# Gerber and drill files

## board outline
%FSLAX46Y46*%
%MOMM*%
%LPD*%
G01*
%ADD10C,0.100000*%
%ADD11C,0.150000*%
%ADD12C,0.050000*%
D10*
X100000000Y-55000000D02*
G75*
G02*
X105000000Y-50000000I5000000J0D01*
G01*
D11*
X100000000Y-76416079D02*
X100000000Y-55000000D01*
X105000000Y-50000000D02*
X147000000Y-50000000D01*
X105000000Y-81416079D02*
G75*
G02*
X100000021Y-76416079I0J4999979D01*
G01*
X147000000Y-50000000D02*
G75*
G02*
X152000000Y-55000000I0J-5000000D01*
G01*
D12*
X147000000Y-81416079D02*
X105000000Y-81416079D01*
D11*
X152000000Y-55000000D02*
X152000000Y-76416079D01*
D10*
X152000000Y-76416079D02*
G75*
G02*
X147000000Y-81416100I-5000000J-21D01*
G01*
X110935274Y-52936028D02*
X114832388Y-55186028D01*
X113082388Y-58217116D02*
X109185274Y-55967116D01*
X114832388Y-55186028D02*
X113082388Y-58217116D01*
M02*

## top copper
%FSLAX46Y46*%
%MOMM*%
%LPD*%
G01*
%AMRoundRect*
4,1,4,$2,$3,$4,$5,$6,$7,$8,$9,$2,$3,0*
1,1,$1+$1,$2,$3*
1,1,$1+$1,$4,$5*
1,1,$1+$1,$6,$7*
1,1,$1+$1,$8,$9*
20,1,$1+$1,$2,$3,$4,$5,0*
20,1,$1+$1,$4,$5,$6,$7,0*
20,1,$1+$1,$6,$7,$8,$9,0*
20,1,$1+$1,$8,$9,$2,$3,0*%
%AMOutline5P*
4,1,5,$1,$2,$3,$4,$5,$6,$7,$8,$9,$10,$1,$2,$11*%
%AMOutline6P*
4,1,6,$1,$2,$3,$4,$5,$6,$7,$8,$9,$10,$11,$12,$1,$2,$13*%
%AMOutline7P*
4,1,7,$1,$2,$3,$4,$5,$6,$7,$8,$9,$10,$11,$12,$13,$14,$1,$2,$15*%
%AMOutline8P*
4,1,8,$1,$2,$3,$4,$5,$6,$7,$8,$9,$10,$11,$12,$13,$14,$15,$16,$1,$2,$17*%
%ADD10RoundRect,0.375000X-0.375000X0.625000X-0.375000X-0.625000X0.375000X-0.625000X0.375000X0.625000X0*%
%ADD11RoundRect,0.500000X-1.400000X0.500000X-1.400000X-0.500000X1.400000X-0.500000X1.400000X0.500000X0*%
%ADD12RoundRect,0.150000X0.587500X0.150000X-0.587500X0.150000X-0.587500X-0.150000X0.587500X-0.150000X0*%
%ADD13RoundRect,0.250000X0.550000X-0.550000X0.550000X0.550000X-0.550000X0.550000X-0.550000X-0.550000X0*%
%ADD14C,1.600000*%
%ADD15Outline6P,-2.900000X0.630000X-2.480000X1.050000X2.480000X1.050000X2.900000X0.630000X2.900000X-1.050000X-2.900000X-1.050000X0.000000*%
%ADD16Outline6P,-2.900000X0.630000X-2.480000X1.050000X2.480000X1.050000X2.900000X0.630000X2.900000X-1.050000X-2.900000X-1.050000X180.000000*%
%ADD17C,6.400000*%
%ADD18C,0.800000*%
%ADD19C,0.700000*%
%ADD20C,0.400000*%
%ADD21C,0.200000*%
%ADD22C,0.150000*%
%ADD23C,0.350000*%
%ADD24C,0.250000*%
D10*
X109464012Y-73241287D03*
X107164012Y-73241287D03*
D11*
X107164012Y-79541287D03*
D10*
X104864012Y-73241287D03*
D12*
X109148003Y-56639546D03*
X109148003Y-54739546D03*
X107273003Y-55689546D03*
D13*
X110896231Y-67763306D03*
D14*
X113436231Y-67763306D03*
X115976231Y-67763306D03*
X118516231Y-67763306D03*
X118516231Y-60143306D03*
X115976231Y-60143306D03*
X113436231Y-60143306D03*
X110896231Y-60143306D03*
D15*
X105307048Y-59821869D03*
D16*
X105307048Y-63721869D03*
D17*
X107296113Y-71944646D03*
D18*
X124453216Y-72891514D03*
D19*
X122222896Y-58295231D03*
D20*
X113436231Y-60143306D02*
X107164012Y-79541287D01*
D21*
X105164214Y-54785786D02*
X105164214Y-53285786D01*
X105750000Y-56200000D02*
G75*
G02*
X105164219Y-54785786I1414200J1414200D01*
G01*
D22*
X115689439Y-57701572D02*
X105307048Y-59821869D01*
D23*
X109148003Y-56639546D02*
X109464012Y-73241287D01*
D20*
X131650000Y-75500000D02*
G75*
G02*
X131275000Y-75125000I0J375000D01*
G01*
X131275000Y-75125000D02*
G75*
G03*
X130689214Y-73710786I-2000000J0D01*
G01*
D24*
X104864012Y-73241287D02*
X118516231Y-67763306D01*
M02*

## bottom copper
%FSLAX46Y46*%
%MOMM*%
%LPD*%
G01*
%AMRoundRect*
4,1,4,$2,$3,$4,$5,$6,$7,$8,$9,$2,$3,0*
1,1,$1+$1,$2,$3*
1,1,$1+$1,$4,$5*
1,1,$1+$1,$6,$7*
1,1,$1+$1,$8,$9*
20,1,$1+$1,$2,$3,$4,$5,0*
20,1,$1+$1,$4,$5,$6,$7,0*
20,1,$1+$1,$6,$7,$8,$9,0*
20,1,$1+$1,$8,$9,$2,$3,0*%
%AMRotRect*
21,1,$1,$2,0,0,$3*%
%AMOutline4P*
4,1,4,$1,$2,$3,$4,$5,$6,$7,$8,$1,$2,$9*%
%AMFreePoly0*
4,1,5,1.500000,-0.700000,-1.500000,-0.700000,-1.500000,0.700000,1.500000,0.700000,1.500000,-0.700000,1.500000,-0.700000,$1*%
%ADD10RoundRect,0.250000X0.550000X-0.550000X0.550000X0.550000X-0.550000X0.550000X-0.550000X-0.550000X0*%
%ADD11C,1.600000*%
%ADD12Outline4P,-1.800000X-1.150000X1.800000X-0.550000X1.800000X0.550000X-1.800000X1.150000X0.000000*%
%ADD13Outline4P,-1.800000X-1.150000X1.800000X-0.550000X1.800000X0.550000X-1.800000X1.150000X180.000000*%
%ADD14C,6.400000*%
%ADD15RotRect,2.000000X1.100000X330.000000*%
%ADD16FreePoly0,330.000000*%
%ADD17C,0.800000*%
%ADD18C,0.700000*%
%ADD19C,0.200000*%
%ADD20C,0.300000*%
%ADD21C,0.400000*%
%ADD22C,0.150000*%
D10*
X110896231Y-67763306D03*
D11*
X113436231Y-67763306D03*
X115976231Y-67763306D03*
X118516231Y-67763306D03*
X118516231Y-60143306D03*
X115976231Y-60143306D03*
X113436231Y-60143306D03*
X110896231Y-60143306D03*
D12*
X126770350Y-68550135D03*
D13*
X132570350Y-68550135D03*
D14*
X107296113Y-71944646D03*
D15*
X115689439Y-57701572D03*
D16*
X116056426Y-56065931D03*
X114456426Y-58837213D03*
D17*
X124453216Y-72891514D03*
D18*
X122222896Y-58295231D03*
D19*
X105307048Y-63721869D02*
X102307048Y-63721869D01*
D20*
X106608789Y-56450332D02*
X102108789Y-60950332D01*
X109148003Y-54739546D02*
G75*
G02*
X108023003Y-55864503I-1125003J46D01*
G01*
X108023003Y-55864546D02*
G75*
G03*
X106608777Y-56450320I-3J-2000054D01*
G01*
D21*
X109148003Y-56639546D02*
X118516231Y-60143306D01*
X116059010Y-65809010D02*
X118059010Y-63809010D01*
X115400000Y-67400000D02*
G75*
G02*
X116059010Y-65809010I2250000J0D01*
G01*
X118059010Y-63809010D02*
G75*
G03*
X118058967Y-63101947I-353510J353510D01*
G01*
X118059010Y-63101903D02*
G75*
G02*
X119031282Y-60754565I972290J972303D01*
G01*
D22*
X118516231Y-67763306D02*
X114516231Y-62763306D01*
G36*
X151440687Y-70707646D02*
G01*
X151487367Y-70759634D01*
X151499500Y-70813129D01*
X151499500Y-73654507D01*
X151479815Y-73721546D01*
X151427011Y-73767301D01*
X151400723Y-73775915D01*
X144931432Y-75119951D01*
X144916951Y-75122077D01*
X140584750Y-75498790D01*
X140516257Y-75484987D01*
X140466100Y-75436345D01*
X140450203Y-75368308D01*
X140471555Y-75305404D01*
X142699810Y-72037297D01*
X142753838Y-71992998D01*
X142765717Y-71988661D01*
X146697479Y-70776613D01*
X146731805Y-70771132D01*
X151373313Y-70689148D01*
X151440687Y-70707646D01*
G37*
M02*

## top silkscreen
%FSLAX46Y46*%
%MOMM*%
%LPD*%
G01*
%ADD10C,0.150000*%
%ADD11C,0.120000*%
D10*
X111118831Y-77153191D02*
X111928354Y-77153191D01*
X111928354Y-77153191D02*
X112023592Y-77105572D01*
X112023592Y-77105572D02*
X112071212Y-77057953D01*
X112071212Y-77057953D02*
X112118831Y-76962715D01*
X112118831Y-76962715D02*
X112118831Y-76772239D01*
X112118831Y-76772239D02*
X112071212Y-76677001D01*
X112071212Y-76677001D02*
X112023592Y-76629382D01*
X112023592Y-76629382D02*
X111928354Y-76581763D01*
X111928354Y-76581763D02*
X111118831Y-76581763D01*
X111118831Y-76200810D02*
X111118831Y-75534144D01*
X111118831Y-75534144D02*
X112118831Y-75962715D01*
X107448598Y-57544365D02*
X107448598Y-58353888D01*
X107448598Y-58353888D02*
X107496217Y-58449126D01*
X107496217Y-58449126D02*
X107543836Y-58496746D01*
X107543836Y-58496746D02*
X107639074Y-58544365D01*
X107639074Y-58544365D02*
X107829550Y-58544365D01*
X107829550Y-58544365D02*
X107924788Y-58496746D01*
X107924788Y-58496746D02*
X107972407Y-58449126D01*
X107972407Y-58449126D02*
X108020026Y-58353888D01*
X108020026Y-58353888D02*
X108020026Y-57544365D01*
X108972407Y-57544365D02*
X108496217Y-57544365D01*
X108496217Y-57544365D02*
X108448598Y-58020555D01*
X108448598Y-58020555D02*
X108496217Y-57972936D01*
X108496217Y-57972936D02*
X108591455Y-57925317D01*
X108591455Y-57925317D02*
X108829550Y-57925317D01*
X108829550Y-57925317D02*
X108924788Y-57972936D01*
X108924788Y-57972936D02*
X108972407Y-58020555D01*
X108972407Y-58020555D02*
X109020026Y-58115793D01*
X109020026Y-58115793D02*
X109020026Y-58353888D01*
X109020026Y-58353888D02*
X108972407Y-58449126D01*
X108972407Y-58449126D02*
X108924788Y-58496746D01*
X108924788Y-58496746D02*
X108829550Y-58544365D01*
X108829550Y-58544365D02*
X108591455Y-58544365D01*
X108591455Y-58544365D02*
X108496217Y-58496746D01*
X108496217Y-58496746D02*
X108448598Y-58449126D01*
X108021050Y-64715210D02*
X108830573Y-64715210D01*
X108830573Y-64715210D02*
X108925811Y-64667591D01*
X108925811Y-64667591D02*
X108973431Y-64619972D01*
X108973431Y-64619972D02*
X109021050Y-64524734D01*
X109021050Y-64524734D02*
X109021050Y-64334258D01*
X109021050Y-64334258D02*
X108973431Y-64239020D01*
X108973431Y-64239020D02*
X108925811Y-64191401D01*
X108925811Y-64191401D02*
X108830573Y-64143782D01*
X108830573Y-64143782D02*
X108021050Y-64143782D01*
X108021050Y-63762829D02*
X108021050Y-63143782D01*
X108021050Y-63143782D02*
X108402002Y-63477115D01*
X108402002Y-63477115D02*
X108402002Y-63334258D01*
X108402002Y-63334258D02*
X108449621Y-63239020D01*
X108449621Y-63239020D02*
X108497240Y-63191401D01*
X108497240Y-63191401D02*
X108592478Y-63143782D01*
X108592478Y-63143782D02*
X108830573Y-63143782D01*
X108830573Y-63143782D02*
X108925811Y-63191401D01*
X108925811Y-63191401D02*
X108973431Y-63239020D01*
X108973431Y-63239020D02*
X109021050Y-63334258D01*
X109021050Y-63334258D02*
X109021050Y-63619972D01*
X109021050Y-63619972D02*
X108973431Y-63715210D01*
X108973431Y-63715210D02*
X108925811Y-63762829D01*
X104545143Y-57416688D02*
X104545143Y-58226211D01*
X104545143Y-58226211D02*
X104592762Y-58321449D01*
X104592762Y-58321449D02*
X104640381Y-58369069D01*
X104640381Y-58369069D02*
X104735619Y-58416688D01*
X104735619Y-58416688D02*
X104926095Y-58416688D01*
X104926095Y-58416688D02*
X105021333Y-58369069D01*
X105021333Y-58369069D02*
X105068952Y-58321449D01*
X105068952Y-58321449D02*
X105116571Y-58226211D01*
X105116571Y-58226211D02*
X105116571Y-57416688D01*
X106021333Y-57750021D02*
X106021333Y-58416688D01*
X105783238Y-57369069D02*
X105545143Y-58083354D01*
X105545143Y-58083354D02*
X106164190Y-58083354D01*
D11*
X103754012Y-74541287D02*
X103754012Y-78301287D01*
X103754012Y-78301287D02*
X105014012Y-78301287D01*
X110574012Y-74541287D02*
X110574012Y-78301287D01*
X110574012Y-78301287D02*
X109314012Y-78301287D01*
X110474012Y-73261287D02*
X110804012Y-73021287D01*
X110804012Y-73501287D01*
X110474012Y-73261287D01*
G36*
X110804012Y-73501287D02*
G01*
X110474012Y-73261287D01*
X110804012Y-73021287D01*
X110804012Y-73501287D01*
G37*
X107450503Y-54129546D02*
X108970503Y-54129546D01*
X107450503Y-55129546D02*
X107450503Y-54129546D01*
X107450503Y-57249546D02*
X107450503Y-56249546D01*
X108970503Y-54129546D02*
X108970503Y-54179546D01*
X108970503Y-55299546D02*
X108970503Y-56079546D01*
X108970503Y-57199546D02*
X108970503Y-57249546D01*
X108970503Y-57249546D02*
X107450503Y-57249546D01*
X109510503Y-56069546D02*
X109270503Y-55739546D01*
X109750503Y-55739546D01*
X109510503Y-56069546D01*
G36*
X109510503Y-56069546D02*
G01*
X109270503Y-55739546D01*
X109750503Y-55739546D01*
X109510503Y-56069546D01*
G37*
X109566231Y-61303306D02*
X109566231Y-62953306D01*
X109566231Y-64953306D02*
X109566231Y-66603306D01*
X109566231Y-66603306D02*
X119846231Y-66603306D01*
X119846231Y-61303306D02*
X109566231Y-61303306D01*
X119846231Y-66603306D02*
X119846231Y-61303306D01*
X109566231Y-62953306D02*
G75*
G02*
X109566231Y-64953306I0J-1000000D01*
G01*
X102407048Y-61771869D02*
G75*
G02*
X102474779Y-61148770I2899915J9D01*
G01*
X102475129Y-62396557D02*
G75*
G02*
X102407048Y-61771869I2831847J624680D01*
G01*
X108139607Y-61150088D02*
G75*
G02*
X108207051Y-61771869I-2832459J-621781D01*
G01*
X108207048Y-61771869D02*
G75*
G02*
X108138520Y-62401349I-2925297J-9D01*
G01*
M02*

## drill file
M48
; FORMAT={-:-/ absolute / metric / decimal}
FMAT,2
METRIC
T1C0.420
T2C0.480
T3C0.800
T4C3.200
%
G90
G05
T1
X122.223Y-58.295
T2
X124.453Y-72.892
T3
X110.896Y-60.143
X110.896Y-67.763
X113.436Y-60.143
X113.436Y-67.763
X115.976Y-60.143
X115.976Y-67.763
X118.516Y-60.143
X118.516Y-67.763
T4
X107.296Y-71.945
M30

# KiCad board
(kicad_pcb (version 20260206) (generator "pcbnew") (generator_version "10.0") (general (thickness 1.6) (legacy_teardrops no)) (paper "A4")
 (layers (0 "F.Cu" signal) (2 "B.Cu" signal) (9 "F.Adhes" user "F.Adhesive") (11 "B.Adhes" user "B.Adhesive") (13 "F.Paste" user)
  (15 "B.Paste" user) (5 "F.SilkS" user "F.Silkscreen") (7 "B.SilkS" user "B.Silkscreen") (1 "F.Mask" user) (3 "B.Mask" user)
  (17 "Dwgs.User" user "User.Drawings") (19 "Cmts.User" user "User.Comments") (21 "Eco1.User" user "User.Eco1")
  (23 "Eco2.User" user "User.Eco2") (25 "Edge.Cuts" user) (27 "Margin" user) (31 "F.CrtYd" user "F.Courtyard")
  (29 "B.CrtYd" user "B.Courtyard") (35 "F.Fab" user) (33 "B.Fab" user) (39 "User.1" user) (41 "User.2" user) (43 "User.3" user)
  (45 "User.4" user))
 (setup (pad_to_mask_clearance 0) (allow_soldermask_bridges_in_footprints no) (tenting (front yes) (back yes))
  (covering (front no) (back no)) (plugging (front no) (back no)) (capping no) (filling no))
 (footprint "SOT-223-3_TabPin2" (layer "F.Cu") (at 107.164012 76.391287 -90)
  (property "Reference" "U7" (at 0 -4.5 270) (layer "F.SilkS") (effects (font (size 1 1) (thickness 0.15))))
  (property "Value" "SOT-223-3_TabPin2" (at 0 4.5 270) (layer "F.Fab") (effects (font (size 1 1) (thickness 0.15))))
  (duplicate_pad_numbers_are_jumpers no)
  (fp_line (start -1.85 3.41) (end 1.91 3.41) (stroke (width 0.12) (type solid)) (layer "F.SilkS"))
  (fp_line (start 1.91 3.41) (end 1.91 2.15) (stroke (width 0.12) (type solid)) (layer "F.SilkS"))
  (fp_line (start -1.85 -3.41) (end 1.91 -3.41) (stroke (width 0.12) (type solid)) (layer "F.SilkS"))
  (fp_line (start 1.91 -3.41) (end 1.91 -2.15) (stroke (width 0.12) (type solid)) (layer "F.SilkS"))
  (fp_poly
   (pts (xy -3.13 -3.31) (xy -3.37 -3.64) (xy -2.89 -3.64) (xy -3.13 -3.31)) (stroke (width 0.12) (type solid)) (fill yes) (layer "F.SilkS"))
  (pad "1" smd roundrect (at -3.15 -2.3 270) (size 2 1.5) (layers "F.Cu" "F.Mask" "F.Paste") (roundrect_rratio 0.25))
  (pad "2" smd roundrect (at -3.15 0 270) (size 2 1.5) (layers "F.Cu" "F.Mask" "F.Paste") (roundrect_rratio 0.25) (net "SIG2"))
  (pad "2" smd roundrect (at 3.15 0 270) (size 2 3.8) (layers "F.Cu" "F.Mask" "F.Paste") (roundrect_rratio 0.25) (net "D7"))
  (pad "3" smd roundrect (at -3.15 2.3 270) (size 2 1.5) (layers "F.Cu" "F.Mask" "F.Paste") (roundrect_rratio 0.25) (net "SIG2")))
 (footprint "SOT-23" (layer "F.Cu") (at 108.210503 55.689546 180)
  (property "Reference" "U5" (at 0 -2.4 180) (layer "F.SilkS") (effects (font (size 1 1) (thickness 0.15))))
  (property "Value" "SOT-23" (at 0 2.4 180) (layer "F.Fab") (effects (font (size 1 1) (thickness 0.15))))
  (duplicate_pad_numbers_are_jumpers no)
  (fp_line (start 0.76 1.56) (end -0.76 1.56) (stroke (width 0.12) (type solid)) (layer "F.SilkS"))
  (fp_line (start 0.76 0.56) (end 0.76 1.56) (stroke (width 0.12) (type solid)) (layer "F.SilkS"))
  (fp_line (start 0.76 -1.56) (end 0.76 -0.56) (stroke (width 0.12) (type solid)) (layer "F.SilkS"))
  (fp_line (start -0.76 1.56) (end -0.76 1.51) (stroke (width 0.12) (type solid)) (layer "F.SilkS"))
  (fp_line (start -0.76 0.39) (end -0.76 -0.39) (stroke (width 0.12) (type solid)) (layer "F.SilkS"))
  (fp_line (start -0.76 -1.51) (end -0.76 -1.56) (stroke (width 0.12) (type solid)) (layer "F.SilkS"))
  (fp_line (start -0.76 -1.56) (end 0.76 -1.56) (stroke (width 0.12) (type solid)) (layer "F.SilkS"))
  (fp_poly (pts (xy -1.3 -0.38) (xy -1.06 -0.05) (xy -1.54 -0.05)) (stroke (width 0.12) (type solid)) (fill yes) (layer "F.SilkS"))
  (pad "1" smd roundrect (at -0.9375 -0.95 180) (size 1.475 0.6) (layers "F.Cu" "F.Mask" "F.Paste") (roundrect_rratio 0.25) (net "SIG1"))
  (pad "2" smd roundrect (at -0.9375 0.95 180) (size 1.475 0.6) (layers "F.Cu" "F.Mask" "F.Paste") (roundrect_rratio 0.25) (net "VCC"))
  (pad "3" smd roundrect (at 0.9375 0 180) (size 1.475 0.6) (layers "F.Cu" "F.Mask" "F.Paste") (roundrect_rratio 0.25) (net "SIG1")))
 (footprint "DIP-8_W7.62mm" (layer "F.Cu") (at 110.896231 67.763306 90)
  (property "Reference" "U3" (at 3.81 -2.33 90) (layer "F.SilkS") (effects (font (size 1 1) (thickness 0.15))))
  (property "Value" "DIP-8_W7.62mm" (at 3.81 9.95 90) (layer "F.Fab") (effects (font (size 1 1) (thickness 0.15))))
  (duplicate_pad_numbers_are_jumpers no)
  (fp_line (start 6.46 -1.33) (end 4.81 -1.33) (stroke (width 0.12) (type solid)) (layer "F.SilkS"))
  (fp_line (start 2.81 -1.33) (end 1.16 -1.33) (stroke (width 0.12) (type solid)) (layer "F.SilkS"))
  (fp_line (start 1.16 -1.33) (end 1.16 8.95) (stroke (width 0.12) (type solid)) (layer "F.SilkS"))
  (fp_line (start 6.46 8.95) (end 6.46 -1.33) (stroke (width 0.12) (type solid)) (layer "F.SilkS"))
  (fp_line (start 1.16 8.95) (end 6.46 8.95) (stroke (width 0.12) (type solid)) (layer "F.SilkS"))
  (fp_arc (start 4.81 -1.33) (mid 3.81 -0.33) (end 2.81 -1.33) (stroke (width 0.12) (type solid)) (layer "F.SilkS"))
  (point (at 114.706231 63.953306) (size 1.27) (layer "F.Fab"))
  (pad "1" thru_hole roundrect (at 0 0 90) (size 1.6 1.6) (drill 0.8) (layers "*.Cu" "*.Mask") (remove_unused_layers no)
   (roundrect_rratio 0.15625))
  (pad "2" thru_hole circle (at 0 2.54 90) (size 1.6 1.6) (drill 0.8) (layers "*.Cu" "*.Mask") (remove_unused_layers no) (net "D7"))
  (pad "3" thru_hole circle (at 0 5.08 90) (size 1.6 1.6) (drill 0.8) (layers "*.Cu" "*.Mask") (remove_unused_layers no) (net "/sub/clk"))
  (pad "4" thru_hole circle (at 0 7.62 90) (size 1.6 1.6) (drill 0.8) (layers "*.Cu" "*.Mask") (remove_unused_layers no) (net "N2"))
  (pad "5" thru_hole circle (at 7.62 7.62 90) (size 1.6 1.6) (drill 0.8) (layers "*.Cu" "*.Mask") (remove_unused_layers no))
  (pad "6" thru_hole circle (at 7.62 5.08 90) (size 1.6 1.6) (drill 0.8) (layers "*.Cu" "*.Mask") (remove_unused_layers no) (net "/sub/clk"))
  (pad "7" thru_hole circle (at 7.62 2.54 90) (size 1.6 1.6) (drill 0.8) (layers "*.Cu" "*.Mask") (remove_unused_layers no))
  (pad "8" thru_hole circle (at 7.62 0 90) (size 1.6 1.6) (drill 0.8) (layers "*.Cu" "*.Mask") (remove_unused_layers no)))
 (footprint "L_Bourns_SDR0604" (layer "F.Cu") (at 105.307048 61.771869)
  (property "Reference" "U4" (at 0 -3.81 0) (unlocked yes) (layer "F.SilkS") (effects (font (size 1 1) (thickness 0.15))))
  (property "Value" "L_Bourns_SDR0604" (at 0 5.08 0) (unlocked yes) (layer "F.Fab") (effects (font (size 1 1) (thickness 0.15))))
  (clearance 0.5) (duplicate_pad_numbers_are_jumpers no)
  (fp_arc (start -2.9 0) (mid -2.883018 -0.313385) (end -2.832269 -0.623099) (stroke (width 0.12) (type default)) (layer "F.SilkS"))
  (fp_arc (start -2.831919 0.624688) (mid -2.88293 0.314193) (end -2.9 0) (stroke (width 0.12) (type default)) (layer "F.SilkS"))
  (fp_arc (start 2.832559 -0.621781) (mid 2.883091 -0.312714) (end 2.9 0) (stroke (width 0.12) (type default)) (layer "F.SilkS"))
  (fp_arc (start 2.9 0) (mid 2.882818 0.3166) (end 2.831472 0.62948) (stroke (width 0.12) (type default)) (layer "F.SilkS"))
  (pad "1" smd roundrect (at 0 -1.95) (size 5.8 2.1) (layers "F.Cu" "F.Mask" "F.Paste") (roundrect_rratio 0) (chamfer_ratio 0.2)
   (chamfer top_left top_right) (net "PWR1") (die_length 2))
  (pad "2" smd roundrect (at 0 1.95 180) (size 5.8 2.1) (layers "F.Cu" "F.Mask" "F.Paste") (roundrect_rratio 0) (chamfer_ratio 0.2)
   (chamfer top_left top_right) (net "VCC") (die_length 2)))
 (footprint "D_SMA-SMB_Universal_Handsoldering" (layer "B.Cu") (at 129.67035 68.550135)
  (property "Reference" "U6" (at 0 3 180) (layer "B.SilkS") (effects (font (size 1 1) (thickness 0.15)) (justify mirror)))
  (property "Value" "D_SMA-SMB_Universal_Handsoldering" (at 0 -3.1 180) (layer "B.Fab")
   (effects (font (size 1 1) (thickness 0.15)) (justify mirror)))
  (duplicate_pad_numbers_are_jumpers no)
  (pad "1" smd trapezoid (at -2.9 0) (size 3.6 1.7) (rect_delta 0.6 0) (layers "B.Cu" "B.Mask" "B.Paste") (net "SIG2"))
  (pad "2" smd trapezoid (at 2.9 0 180) (size 3.6 1.7) (rect_delta 0.6 0) (layers "B.Cu" "B.Mask" "B.Paste") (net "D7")))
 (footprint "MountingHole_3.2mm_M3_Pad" (layer "B.Cu") (at 107.296113 71.944646)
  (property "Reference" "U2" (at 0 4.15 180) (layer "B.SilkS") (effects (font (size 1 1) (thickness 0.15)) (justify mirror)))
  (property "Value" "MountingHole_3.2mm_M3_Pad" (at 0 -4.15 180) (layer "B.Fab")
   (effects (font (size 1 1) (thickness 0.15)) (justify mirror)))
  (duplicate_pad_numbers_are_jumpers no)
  (pad "1" thru_hole circle (at 0 0) (size 6.4 6.4) (drill 3.2) (layers "*.Cu" "*.Mask") (remove_unused_layers no) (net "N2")
   (zone_connect 2)))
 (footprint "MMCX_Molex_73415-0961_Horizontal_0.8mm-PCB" (layer "B.Cu") (at 113.307869 56.326572 -30)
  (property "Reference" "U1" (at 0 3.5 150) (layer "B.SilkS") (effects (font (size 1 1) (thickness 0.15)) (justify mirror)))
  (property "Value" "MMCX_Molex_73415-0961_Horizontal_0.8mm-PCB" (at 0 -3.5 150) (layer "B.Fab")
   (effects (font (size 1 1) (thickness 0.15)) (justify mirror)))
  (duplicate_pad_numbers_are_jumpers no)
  (fp_line (start -3.75 -1.75) (end 0.75 -1.75) (stroke (width 0.1) (type solid)) (layer "Edge.Cuts"))
  (fp_line (start 0.75 1.75) (end -3.75 1.749999) (stroke (width 0.1) (type solid)) (layer "Edge.Cuts"))
  (fp_line (start 0.75 -1.75) (end 0.75 1.75) (stroke (width 0.1) (type solid)) (layer "Edge.Cuts"))
  (pad "1" smd rect (at 2.75 0 330) (size 2 1.1) (layers "B.Cu" "B.Mask" "B.Paste") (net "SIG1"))
  (pad "2" smd custom (at 2.25 -1.6 330) (size 3 1.4) (layers "B.Cu" "B.Mask" "B.Paste") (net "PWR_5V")
   (options (clearance outline) (anchor rect)) (primitives))
  (pad "2" smd custom (at 2.25 1.6 330) (size 3 1.4) (layers "B.Cu" "B.Mask" "B.Paste") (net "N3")
   (options (clearance outline) (anchor rect)) (primitives)))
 (gr_arc (start 100 55) (mid 101.464466 51.464466) (end 105 50) (stroke (width 0.1) (type default)) (layer "Edge.Cuts"))
 (gr_line (start 100 76.416079) (end 100 55) (stroke (width 0.15) (type default)) (layer "Edge.Cuts"))
 (gr_line (start 105 50) (end 147 50) (stroke (width 0.15) (type default)) (layer "Edge.Cuts"))
 (gr_arc (start 105 81.416079) (mid 101.464466 79.951612) (end 100 76.416079) (stroke (width 0.15) (type default)) (layer "Edge.Cuts"))
 (gr_arc (start 147 50) (mid 150.535533 51.464466) (end 152 55) (stroke (width 0.15) (type default)) (layer "Edge.Cuts"))
 (gr_line (start 147 81.416079) (end 105 81.416079) (stroke (width 0.05) (type default)) (layer "Edge.Cuts"))
 (gr_line (start 152 55) (end 152 76.416079) (stroke (width 0.15) (type default)) (layer "Edge.Cuts"))
 (gr_arc (start 152 76.416079) (mid 150.535533 79.951612) (end 147 81.416079) (stroke (width 0.1) (type default)) (layer "Edge.Cuts"))
 (segment (start 113.436231 60.143306) (end 107.164012 79.541287) (width 0.4) (layer "F.Cu") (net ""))
 (segment (start 105.307048 63.721869) (end 102.307048 63.721869) (width 0.2) (layer "B.Cu") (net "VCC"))
 (segment (start 106.608789 56.450332) (end 102.108789 60.950332) (width 0.3) (layer "B.Cu") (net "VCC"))
 (arc (start 109.148003 54.739546) (mid 108.818498 55.535041) (end 108.023003 55.864546) (width 0.3) (layer "B.Cu") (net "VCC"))
 (arc (start 108.023003 55.864546) (mid 107.257636 56.016787) (end 106.608789 56.450332) (width 0.3) (locked yes) (layer "B.Cu") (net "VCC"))
 (segment (start 105.164214 54.785786) (end 105.164214 53.285786) (width 0.2) (layer "F.Cu") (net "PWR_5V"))
 (arc (start 105.75 56.2) (mid 105.316454 55.551153) (end 105.164214 54.785786) (width 0.2) (layer "F.Cu") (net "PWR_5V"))
 (segment (start 115.689439 57.701572) (end 105.307048 59.821869) (width 0.15) (layer "F.Cu") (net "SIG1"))
 (segment (start 109.148003 56.639546) (end 109.464012 73.241287) (width 0.35) (layer "F.Cu") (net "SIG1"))
 (segment (start 109.148003 56.639546) (end 118.516231 60.143306) (width 0.4) (layer "B.Cu") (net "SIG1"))
 (via (at 124.453216 72.891514) (size 0.8) (drill 0.48) (layers "F.Cu" "B.Cu") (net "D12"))
 (segment (start 116.05901 65.80901) (end 118.05901 63.80901) (width 0.4) (layer "B.Cu") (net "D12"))
 (arc (start 115.4 67.4) (mid 115.571271 66.538962) (end 116.05901 65.80901) (width 0.4) (layer "B.Cu") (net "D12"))
 (arc (start 118.05901 63.80901) (mid 118.205457 63.455457) (end 118.05901 63.101903) (width 0.4) (layer "B.Cu") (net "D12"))
 (arc (start 118.05901 63.101903) (mid 117.760947 61.603441) (end 119.031282 60.754631) (width 0.4) (layer "B.Cu") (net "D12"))
 (via (at 122.222896 58.295231) (size 0.7) (drill 0.42) (layers "F.Cu" "B.Cu") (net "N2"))
 (arc (start 131.65 75.5) (mid 131.384835 75.390165) (end 131.275 75.125) (width 0.4) (layer "F.Cu") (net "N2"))
 (arc (start 131.275 75.125) (mid 131.122759 74.359633) (end 130.689214 73.710786) (width 0.4) (layer "F.Cu") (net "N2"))
 (segment (start 118.516231 67.763306) (end 114.516231 62.763306) (width 0.15) (layer "B.Cu") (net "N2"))
 (segment (start 104.864012 73.241287) (end 118.516231 67.763306) (width 0.25) (layer "F.Cu") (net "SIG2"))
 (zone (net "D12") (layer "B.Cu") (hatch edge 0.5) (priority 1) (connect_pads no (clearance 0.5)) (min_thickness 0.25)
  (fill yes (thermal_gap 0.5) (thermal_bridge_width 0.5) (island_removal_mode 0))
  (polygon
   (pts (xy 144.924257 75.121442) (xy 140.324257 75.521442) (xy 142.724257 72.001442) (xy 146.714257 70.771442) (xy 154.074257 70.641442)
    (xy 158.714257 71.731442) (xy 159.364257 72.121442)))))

